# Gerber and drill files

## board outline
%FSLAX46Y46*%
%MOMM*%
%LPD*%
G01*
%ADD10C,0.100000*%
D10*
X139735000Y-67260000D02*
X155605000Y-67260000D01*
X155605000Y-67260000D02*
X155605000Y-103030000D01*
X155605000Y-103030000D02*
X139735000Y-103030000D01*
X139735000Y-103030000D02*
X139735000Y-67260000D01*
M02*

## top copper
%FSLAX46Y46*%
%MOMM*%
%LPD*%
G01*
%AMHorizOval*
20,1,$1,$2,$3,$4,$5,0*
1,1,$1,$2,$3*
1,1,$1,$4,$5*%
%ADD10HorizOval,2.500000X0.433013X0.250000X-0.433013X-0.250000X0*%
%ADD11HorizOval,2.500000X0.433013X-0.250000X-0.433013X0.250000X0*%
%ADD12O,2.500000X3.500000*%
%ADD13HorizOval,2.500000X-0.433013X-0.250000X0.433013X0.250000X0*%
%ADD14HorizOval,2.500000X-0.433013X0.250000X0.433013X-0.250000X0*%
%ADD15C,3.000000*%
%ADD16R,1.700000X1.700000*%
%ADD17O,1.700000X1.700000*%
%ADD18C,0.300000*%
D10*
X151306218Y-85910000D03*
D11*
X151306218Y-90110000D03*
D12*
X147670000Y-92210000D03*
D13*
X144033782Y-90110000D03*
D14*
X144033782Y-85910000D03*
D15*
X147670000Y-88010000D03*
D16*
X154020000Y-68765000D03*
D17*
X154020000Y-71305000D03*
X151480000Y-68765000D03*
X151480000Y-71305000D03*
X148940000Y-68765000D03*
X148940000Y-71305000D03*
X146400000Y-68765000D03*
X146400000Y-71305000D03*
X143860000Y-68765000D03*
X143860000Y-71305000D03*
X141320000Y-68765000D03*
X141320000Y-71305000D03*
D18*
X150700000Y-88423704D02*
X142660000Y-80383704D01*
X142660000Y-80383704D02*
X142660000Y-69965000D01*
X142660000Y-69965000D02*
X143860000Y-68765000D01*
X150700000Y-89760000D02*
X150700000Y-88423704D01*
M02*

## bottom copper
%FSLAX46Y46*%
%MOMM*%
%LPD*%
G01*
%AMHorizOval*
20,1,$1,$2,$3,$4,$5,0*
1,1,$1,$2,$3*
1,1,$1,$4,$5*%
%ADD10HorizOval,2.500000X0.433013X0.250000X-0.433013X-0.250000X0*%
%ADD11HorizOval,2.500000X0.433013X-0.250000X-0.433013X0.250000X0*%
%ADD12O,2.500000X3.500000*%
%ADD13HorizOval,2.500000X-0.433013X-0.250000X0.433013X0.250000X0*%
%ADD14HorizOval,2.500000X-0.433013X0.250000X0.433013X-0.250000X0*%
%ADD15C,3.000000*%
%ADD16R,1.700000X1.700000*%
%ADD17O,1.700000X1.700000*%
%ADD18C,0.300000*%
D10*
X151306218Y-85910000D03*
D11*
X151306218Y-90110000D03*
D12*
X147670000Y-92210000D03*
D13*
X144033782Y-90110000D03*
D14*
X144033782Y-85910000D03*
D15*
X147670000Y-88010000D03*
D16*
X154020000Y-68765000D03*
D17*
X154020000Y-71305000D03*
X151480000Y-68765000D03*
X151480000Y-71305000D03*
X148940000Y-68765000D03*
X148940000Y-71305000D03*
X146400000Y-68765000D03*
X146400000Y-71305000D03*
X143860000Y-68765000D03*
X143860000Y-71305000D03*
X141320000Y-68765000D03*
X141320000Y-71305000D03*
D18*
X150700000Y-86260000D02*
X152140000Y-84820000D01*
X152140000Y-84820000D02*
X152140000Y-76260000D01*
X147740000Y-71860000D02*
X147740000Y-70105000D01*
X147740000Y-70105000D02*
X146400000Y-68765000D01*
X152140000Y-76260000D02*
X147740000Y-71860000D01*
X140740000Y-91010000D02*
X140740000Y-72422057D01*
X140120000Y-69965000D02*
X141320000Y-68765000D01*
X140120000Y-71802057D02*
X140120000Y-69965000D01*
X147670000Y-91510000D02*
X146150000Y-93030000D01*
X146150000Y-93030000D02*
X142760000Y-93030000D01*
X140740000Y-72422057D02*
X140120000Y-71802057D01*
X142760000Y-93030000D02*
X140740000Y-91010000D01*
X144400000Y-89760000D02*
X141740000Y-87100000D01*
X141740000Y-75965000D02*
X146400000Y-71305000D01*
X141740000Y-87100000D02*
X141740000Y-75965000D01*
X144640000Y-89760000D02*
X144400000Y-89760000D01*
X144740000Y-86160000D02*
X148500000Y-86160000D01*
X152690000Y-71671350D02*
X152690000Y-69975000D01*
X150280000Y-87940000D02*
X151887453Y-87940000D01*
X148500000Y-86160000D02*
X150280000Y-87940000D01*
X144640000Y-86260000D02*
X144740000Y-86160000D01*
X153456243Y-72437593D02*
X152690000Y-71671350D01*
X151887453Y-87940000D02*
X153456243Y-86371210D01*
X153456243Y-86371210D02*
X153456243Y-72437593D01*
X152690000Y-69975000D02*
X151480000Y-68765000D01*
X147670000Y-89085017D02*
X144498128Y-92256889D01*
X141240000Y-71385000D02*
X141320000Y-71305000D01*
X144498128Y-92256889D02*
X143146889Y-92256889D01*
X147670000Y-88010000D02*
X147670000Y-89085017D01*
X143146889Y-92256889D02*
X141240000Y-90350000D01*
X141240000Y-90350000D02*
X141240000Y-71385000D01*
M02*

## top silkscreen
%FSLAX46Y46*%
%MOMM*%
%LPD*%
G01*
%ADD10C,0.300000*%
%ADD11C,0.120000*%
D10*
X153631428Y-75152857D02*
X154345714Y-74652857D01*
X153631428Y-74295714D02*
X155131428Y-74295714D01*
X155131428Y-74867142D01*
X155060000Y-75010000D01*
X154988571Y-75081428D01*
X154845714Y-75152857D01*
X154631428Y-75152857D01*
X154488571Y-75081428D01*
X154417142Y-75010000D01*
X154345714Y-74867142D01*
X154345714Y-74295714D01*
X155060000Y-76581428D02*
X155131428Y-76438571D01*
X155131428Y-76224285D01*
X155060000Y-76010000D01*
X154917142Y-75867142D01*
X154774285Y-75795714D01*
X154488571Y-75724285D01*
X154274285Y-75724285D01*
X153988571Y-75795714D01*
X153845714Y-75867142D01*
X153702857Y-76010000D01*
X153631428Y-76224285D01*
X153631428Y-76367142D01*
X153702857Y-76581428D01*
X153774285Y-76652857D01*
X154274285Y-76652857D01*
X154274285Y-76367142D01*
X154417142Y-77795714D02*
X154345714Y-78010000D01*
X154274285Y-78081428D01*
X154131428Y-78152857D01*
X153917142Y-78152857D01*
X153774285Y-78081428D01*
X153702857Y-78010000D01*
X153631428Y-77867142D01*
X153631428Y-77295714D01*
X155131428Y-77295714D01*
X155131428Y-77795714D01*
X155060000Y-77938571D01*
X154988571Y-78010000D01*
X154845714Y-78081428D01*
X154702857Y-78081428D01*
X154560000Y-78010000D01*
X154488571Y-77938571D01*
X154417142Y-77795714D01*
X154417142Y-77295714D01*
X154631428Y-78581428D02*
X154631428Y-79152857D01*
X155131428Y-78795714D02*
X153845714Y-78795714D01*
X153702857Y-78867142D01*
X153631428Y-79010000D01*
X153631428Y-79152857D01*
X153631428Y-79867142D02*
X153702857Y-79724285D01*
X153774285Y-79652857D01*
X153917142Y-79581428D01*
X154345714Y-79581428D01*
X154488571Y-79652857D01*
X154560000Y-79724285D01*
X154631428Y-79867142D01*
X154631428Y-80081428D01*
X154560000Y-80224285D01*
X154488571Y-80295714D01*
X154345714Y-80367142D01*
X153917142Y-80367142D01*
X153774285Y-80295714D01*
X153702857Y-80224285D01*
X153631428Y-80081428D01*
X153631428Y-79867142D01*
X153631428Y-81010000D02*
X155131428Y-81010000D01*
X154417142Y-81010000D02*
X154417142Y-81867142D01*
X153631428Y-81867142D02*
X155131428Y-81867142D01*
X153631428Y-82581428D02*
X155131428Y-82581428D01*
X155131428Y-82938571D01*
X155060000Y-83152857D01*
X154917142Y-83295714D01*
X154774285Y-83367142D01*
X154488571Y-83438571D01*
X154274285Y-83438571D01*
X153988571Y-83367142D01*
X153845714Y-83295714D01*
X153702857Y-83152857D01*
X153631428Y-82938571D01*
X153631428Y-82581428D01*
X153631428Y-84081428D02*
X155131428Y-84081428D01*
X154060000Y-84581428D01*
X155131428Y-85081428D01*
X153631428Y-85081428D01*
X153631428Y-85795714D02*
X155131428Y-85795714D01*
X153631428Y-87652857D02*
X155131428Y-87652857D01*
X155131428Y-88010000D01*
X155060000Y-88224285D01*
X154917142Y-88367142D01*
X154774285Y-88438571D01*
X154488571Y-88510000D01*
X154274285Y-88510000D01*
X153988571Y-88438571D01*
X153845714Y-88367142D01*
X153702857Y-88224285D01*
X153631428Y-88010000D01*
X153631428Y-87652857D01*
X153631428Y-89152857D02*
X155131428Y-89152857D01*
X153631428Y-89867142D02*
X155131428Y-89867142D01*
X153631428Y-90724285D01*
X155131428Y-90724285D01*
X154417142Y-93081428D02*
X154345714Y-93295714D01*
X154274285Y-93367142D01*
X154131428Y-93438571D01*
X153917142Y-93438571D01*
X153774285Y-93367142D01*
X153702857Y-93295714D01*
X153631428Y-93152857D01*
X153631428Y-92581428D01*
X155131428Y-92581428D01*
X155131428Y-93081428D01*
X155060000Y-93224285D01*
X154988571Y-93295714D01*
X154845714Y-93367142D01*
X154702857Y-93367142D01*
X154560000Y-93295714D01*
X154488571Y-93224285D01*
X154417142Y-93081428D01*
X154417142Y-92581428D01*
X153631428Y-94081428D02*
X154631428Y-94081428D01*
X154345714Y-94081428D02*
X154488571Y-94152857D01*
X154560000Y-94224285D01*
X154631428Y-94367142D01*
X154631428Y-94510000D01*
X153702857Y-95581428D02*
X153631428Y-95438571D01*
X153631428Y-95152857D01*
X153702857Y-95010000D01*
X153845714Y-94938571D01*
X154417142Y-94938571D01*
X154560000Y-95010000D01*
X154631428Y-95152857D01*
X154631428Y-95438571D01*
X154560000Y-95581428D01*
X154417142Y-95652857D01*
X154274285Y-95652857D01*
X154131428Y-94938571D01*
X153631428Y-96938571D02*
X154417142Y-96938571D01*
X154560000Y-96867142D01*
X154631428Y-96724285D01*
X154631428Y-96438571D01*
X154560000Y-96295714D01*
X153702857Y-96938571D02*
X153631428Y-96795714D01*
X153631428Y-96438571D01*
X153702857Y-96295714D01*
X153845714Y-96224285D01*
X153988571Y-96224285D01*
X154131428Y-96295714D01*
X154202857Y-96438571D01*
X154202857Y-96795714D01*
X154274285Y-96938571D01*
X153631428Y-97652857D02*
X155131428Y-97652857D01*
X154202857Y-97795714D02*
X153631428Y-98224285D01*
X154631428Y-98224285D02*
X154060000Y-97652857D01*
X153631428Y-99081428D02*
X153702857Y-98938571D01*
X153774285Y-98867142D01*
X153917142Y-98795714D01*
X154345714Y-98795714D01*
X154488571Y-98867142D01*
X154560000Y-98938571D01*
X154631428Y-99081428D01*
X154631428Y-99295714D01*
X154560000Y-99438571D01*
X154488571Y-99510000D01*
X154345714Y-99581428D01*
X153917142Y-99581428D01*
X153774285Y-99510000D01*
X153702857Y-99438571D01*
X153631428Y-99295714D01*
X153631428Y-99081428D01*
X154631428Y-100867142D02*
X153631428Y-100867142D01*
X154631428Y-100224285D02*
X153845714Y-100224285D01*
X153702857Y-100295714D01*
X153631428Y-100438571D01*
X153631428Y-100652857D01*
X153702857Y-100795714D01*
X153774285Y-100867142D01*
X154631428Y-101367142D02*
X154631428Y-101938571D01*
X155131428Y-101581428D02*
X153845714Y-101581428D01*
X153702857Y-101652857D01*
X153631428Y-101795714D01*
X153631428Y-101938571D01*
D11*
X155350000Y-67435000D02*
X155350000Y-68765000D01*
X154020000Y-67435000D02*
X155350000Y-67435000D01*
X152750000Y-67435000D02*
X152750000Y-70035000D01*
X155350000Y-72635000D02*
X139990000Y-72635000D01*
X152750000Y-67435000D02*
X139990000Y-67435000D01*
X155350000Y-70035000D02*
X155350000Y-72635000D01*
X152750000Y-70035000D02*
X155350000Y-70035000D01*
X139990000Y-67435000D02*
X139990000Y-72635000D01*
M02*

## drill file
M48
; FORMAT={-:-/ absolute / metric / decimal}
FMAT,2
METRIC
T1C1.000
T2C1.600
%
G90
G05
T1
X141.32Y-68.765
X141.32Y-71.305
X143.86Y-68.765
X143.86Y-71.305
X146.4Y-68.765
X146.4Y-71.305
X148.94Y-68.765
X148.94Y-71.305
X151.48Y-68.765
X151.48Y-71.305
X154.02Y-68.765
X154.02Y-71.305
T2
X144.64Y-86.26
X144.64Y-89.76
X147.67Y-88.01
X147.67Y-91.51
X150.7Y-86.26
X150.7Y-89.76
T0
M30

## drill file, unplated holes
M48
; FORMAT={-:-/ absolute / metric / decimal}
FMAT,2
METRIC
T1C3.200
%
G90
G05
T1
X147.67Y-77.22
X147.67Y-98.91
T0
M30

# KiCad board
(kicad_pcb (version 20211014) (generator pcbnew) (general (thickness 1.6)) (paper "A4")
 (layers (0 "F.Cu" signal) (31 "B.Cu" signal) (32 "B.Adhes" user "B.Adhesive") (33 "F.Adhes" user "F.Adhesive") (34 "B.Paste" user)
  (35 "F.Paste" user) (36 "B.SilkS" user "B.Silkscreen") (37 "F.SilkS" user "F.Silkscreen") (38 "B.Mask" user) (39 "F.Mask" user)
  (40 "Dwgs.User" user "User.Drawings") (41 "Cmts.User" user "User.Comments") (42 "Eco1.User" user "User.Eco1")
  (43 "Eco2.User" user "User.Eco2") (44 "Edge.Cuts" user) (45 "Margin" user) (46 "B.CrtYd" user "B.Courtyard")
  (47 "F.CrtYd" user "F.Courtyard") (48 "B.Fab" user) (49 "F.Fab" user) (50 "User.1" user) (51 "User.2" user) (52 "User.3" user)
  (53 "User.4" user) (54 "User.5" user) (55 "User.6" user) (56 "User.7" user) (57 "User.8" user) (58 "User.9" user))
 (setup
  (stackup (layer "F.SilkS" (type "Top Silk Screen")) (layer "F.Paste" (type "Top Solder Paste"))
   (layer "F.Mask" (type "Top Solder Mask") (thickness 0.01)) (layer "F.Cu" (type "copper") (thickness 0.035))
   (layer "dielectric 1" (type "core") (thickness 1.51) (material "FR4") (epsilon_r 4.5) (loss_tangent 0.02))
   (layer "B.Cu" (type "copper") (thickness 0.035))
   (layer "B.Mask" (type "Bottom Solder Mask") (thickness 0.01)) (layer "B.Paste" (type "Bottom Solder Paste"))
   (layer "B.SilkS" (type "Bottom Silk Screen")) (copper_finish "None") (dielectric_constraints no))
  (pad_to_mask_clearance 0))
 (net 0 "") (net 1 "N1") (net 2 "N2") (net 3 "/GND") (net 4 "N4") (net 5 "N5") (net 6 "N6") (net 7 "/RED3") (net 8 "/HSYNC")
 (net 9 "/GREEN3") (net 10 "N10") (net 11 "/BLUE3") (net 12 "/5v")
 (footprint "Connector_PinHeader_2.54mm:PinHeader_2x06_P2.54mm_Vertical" (layer "F.Cu") (at 154.02 68.765 -90)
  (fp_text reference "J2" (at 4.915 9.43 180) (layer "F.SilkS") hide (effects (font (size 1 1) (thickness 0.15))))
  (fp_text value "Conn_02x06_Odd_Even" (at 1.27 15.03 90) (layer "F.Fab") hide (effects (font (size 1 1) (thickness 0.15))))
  (fp_line (start -1.33 -1.33) (end 0 -1.33) (layer "F.SilkS") (width 0.12))
  (fp_line (start -1.33 0) (end -1.33 -1.33) (layer "F.SilkS") (width 0.12))
  (fp_line (start -1.33 1.27) (end 1.27 1.27) (layer "F.SilkS") (width 0.12))
  (fp_line (start 3.87 -1.33) (end 3.87 14.03) (layer "F.SilkS") (width 0.12))
  (fp_line (start -1.33 1.27) (end -1.33 14.03) (layer "F.SilkS") (width 0.12))
  (fp_line (start 1.27 -1.33) (end 3.87 -1.33) (layer "F.SilkS") (width 0.12))
  (fp_line (start 1.27 1.27) (end 1.27 -1.33) (layer "F.SilkS") (width 0.12))
  (fp_line (start -1.33 14.03) (end 3.87 14.03) (layer "F.SilkS") (width 0.12))
  (pad "1" thru_hole rect (at 0 0 270) (size 1.7 1.7) (drill 1) (layers *.Cu *.Mask) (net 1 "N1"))
  (pad "2" thru_hole oval (at 2.54 0 270) (size 1.7 1.7) (drill 1) (layers *.Cu *.Mask) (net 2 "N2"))
  (pad "3" thru_hole oval (at 0 2.54 270) (size 1.7 1.7) (drill 1) (layers *.Cu *.Mask) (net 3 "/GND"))
  (pad "4" thru_hole oval (at 2.54 2.54 270) (size 1.7 1.7) (drill 1) (layers *.Cu *.Mask) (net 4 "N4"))
  (pad "5" thru_hole oval (at 0 5.08 270) (size 1.7 1.7) (drill 1) (layers *.Cu *.Mask) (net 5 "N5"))
  (pad "6" thru_hole oval (at 2.54 5.08 270) (size 1.7 1.7) (drill 1) (layers *.Cu *.Mask) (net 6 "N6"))
  (pad "7" thru_hole oval (at 0 7.62 270) (size 1.7 1.7) (drill 1) (layers *.Cu *.Mask) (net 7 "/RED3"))
  (pad "8" thru_hole oval (at 2.54 7.62 270) (size 1.7 1.7) (drill 1) (layers *.Cu *.Mask) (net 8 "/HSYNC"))
  (pad "9" thru_hole oval (at 0 10.16 270) (size 1.7 1.7) (drill 1) (layers *.Cu *.Mask) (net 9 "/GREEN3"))
  (pad "10" thru_hole oval (at 2.54 10.16 270) (size 1.7 1.7) (drill 1) (layers *.Cu *.Mask) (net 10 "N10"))
  (pad "11" thru_hole oval (at 0 12.7 270) (size 1.7 1.7) (drill 1) (layers *.Cu *.Mask) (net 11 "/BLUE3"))
  (pad "12" thru_hole oval (at 2.54 12.7 270) (size 1.7 1.7) (drill 1) (layers *.Cu *.Mask) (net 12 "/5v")))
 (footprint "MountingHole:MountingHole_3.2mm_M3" (layer "F.Cu") (at 147.67 98.91)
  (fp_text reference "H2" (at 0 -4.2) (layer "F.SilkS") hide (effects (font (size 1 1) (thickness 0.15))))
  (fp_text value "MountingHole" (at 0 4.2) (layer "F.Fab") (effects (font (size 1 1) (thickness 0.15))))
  (pad "" np_thru_hole circle (at 0 0) (size 3.2 3.2) (drill 3.2) (layers *.Cu *.Mask)))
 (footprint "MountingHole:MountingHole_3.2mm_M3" (layer "F.Cu") (at 147.67 77.22)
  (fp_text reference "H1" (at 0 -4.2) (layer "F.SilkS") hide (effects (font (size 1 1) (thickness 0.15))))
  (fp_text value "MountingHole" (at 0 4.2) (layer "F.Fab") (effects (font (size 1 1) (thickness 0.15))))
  (pad "" np_thru_hole circle (at 0 0) (size 3.2 3.2) (drill 3.2) (layers *.Cu *.Mask)))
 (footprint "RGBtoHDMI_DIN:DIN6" (layer "B.Cu") (at 147.67 88.01)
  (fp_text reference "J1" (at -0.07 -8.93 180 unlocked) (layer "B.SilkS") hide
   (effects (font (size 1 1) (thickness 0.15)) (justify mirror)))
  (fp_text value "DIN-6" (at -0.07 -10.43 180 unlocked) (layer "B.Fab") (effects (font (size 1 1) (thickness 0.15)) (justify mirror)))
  (pad "1" thru_hole oval (at 3.03 -1.75 30) (size 3.5 2.5) (drill 1.6 (offset 0.7 0)) (layers *.Cu *.Mask) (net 7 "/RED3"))
  (pad "2" thru_hole oval (at 3.03 1.75 330) (size 3.5 2.5) (drill 1.6 (offset 0.7 0)) (layers *.Cu *.Mask) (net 9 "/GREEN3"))
  (pad "3" thru_hole oval (at 0 3.5 270) (size 3.5 2.5) (drill 1.6 (offset 0.7 0)) (layers *.Cu *.Mask) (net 11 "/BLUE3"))
  (pad "4" thru_hole oval (at -3.03 1.75 210) (size 3.5 2.5) (drill 1.6 (offset 0.7 0)) (layers *.Cu *.Mask) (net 8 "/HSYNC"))
  (pad "5" thru_hole oval (at -3.03 -1.75 150) (size 3.5 2.5) (drill 1.6 (offset 0.7 0)) (layers *.Cu *.Mask) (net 3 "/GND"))
  (pad "6" thru_hole circle (at 0 0 30) (size 3 3) (drill 1.6) (layers *.Cu *.Mask) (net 12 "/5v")))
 (gr_rect (start 139.735 67.26) (end 155.605 103.03) (layer "Edge.Cuts") (width 0.1) (fill none))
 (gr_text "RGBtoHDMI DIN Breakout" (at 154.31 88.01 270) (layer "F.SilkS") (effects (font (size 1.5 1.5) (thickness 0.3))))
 (segment (start 150.7 86.26) (end 152.14 84.82) (width 0.3) (layer "B.Cu") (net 7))
 (segment (start 152.14 84.82) (end 152.14 76.26) (width 0.3) (layer "B.Cu") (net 7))
 (segment (start 147.74 71.86) (end 147.74 70.105) (width 0.3) (layer "B.Cu") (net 7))
 (segment (start 147.74 70.105) (end 146.4 68.765) (width 0.3) (layer "B.Cu") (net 7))
 (segment (start 152.14 76.26) (end 147.74 71.86) (width 0.3) (layer "B.Cu") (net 7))
 (segment (start 150.7 88.423704) (end 142.66 80.383704) (width 0.3) (layer "F.Cu") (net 9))
 (segment (start 142.66 80.383704) (end 142.66 69.965) (width 0.3) (layer "F.Cu") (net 9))
 (segment (start 142.66 69.965) (end 143.86 68.765) (width 0.3) (layer "F.Cu") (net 9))
 (segment (start 150.7 89.76) (end 150.7 88.423704) (width 0.3) (layer "F.Cu") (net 9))
 (segment (start 140.74 91.01) (end 140.74 72.422057) (width 0.3) (layer "B.Cu") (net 11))
 (segment (start 140.12 69.965) (end 141.32 68.765) (width 0.3) (layer "B.Cu") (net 11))
 (segment (start 140.12 71.802057) (end 140.12 69.965) (width 0.3) (layer "B.Cu") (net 11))
 (segment (start 147.67 91.51) (end 146.15 93.03) (width 0.3) (layer "B.Cu") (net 11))
 (segment (start 146.15 93.03) (end 142.76 93.03) (width 0.3) (layer "B.Cu") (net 11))
 (segment (start 140.74 72.422057) (end 140.12 71.802057) (width 0.3) (layer "B.Cu") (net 11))
 (segment (start 142.76 93.03) (end 140.74 91.01) (width 0.3) (layer "B.Cu") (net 11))
 (segment (start 144.4 89.76) (end 141.74 87.1) (width 0.3) (layer "B.Cu") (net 8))
 (segment (start 141.74 75.965) (end 146.4 71.305) (width 0.3) (layer "B.Cu") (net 8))
 (segment (start 141.74 87.1) (end 141.74 75.965) (width 0.3) (layer "B.Cu") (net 8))
 (segment (start 144.64 89.76) (end 144.4 89.76) (width 0.3) (layer "B.Cu") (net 8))
 (segment (start 144.74 86.16) (end 148.5 86.16) (width 0.3) (layer "B.Cu") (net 3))
 (segment (start 152.69 71.67135) (end 152.69 69.975) (width 0.3) (layer "B.Cu") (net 3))
 (segment (start 150.28 87.94) (end 151.887453 87.94) (width 0.3) (layer "B.Cu") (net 3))
 (segment (start 148.5 86.16) (end 150.28 87.94) (width 0.3) (layer "B.Cu") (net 3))
 (segment (start 144.64 86.26) (end 144.74 86.16) (width 0.3) (layer "B.Cu") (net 3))
 (segment (start 153.456243 72.437593) (end 152.69 71.67135) (width 0.3) (layer "B.Cu") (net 3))
 (segment (start 151.887453 87.94) (end 153.456243 86.37121) (width 0.3) (layer "B.Cu") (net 3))
 (segment (start 153.456243 86.37121) (end 153.456243 72.437593) (width 0.3) (layer "B.Cu") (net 3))
 (segment (start 152.69 69.975) (end 151.48 68.765) (width 0.3) (layer "B.Cu") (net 3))
 (segment (start 147.67 89.085017) (end 144.498128 92.256889) (width 0.3) (layer "B.Cu") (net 12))
 (segment (start 141.24 71.385) (end 141.32 71.305) (width 0.3) (layer "B.Cu") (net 12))
 (segment (start 144.498128 92.256889) (end 143.146889 92.256889) (width 0.3) (layer "B.Cu") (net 12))
 (segment (start 147.67 88.01) (end 147.67 89.085017) (width 0.3) (layer "B.Cu") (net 12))
 (segment (start 143.146889 92.256889) (end 141.24 90.35) (width 0.3) (layer "B.Cu") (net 12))
 (segment (start 141.24 90.35) (end 141.24 71.385) (width 0.3) (layer "B.Cu") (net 12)))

